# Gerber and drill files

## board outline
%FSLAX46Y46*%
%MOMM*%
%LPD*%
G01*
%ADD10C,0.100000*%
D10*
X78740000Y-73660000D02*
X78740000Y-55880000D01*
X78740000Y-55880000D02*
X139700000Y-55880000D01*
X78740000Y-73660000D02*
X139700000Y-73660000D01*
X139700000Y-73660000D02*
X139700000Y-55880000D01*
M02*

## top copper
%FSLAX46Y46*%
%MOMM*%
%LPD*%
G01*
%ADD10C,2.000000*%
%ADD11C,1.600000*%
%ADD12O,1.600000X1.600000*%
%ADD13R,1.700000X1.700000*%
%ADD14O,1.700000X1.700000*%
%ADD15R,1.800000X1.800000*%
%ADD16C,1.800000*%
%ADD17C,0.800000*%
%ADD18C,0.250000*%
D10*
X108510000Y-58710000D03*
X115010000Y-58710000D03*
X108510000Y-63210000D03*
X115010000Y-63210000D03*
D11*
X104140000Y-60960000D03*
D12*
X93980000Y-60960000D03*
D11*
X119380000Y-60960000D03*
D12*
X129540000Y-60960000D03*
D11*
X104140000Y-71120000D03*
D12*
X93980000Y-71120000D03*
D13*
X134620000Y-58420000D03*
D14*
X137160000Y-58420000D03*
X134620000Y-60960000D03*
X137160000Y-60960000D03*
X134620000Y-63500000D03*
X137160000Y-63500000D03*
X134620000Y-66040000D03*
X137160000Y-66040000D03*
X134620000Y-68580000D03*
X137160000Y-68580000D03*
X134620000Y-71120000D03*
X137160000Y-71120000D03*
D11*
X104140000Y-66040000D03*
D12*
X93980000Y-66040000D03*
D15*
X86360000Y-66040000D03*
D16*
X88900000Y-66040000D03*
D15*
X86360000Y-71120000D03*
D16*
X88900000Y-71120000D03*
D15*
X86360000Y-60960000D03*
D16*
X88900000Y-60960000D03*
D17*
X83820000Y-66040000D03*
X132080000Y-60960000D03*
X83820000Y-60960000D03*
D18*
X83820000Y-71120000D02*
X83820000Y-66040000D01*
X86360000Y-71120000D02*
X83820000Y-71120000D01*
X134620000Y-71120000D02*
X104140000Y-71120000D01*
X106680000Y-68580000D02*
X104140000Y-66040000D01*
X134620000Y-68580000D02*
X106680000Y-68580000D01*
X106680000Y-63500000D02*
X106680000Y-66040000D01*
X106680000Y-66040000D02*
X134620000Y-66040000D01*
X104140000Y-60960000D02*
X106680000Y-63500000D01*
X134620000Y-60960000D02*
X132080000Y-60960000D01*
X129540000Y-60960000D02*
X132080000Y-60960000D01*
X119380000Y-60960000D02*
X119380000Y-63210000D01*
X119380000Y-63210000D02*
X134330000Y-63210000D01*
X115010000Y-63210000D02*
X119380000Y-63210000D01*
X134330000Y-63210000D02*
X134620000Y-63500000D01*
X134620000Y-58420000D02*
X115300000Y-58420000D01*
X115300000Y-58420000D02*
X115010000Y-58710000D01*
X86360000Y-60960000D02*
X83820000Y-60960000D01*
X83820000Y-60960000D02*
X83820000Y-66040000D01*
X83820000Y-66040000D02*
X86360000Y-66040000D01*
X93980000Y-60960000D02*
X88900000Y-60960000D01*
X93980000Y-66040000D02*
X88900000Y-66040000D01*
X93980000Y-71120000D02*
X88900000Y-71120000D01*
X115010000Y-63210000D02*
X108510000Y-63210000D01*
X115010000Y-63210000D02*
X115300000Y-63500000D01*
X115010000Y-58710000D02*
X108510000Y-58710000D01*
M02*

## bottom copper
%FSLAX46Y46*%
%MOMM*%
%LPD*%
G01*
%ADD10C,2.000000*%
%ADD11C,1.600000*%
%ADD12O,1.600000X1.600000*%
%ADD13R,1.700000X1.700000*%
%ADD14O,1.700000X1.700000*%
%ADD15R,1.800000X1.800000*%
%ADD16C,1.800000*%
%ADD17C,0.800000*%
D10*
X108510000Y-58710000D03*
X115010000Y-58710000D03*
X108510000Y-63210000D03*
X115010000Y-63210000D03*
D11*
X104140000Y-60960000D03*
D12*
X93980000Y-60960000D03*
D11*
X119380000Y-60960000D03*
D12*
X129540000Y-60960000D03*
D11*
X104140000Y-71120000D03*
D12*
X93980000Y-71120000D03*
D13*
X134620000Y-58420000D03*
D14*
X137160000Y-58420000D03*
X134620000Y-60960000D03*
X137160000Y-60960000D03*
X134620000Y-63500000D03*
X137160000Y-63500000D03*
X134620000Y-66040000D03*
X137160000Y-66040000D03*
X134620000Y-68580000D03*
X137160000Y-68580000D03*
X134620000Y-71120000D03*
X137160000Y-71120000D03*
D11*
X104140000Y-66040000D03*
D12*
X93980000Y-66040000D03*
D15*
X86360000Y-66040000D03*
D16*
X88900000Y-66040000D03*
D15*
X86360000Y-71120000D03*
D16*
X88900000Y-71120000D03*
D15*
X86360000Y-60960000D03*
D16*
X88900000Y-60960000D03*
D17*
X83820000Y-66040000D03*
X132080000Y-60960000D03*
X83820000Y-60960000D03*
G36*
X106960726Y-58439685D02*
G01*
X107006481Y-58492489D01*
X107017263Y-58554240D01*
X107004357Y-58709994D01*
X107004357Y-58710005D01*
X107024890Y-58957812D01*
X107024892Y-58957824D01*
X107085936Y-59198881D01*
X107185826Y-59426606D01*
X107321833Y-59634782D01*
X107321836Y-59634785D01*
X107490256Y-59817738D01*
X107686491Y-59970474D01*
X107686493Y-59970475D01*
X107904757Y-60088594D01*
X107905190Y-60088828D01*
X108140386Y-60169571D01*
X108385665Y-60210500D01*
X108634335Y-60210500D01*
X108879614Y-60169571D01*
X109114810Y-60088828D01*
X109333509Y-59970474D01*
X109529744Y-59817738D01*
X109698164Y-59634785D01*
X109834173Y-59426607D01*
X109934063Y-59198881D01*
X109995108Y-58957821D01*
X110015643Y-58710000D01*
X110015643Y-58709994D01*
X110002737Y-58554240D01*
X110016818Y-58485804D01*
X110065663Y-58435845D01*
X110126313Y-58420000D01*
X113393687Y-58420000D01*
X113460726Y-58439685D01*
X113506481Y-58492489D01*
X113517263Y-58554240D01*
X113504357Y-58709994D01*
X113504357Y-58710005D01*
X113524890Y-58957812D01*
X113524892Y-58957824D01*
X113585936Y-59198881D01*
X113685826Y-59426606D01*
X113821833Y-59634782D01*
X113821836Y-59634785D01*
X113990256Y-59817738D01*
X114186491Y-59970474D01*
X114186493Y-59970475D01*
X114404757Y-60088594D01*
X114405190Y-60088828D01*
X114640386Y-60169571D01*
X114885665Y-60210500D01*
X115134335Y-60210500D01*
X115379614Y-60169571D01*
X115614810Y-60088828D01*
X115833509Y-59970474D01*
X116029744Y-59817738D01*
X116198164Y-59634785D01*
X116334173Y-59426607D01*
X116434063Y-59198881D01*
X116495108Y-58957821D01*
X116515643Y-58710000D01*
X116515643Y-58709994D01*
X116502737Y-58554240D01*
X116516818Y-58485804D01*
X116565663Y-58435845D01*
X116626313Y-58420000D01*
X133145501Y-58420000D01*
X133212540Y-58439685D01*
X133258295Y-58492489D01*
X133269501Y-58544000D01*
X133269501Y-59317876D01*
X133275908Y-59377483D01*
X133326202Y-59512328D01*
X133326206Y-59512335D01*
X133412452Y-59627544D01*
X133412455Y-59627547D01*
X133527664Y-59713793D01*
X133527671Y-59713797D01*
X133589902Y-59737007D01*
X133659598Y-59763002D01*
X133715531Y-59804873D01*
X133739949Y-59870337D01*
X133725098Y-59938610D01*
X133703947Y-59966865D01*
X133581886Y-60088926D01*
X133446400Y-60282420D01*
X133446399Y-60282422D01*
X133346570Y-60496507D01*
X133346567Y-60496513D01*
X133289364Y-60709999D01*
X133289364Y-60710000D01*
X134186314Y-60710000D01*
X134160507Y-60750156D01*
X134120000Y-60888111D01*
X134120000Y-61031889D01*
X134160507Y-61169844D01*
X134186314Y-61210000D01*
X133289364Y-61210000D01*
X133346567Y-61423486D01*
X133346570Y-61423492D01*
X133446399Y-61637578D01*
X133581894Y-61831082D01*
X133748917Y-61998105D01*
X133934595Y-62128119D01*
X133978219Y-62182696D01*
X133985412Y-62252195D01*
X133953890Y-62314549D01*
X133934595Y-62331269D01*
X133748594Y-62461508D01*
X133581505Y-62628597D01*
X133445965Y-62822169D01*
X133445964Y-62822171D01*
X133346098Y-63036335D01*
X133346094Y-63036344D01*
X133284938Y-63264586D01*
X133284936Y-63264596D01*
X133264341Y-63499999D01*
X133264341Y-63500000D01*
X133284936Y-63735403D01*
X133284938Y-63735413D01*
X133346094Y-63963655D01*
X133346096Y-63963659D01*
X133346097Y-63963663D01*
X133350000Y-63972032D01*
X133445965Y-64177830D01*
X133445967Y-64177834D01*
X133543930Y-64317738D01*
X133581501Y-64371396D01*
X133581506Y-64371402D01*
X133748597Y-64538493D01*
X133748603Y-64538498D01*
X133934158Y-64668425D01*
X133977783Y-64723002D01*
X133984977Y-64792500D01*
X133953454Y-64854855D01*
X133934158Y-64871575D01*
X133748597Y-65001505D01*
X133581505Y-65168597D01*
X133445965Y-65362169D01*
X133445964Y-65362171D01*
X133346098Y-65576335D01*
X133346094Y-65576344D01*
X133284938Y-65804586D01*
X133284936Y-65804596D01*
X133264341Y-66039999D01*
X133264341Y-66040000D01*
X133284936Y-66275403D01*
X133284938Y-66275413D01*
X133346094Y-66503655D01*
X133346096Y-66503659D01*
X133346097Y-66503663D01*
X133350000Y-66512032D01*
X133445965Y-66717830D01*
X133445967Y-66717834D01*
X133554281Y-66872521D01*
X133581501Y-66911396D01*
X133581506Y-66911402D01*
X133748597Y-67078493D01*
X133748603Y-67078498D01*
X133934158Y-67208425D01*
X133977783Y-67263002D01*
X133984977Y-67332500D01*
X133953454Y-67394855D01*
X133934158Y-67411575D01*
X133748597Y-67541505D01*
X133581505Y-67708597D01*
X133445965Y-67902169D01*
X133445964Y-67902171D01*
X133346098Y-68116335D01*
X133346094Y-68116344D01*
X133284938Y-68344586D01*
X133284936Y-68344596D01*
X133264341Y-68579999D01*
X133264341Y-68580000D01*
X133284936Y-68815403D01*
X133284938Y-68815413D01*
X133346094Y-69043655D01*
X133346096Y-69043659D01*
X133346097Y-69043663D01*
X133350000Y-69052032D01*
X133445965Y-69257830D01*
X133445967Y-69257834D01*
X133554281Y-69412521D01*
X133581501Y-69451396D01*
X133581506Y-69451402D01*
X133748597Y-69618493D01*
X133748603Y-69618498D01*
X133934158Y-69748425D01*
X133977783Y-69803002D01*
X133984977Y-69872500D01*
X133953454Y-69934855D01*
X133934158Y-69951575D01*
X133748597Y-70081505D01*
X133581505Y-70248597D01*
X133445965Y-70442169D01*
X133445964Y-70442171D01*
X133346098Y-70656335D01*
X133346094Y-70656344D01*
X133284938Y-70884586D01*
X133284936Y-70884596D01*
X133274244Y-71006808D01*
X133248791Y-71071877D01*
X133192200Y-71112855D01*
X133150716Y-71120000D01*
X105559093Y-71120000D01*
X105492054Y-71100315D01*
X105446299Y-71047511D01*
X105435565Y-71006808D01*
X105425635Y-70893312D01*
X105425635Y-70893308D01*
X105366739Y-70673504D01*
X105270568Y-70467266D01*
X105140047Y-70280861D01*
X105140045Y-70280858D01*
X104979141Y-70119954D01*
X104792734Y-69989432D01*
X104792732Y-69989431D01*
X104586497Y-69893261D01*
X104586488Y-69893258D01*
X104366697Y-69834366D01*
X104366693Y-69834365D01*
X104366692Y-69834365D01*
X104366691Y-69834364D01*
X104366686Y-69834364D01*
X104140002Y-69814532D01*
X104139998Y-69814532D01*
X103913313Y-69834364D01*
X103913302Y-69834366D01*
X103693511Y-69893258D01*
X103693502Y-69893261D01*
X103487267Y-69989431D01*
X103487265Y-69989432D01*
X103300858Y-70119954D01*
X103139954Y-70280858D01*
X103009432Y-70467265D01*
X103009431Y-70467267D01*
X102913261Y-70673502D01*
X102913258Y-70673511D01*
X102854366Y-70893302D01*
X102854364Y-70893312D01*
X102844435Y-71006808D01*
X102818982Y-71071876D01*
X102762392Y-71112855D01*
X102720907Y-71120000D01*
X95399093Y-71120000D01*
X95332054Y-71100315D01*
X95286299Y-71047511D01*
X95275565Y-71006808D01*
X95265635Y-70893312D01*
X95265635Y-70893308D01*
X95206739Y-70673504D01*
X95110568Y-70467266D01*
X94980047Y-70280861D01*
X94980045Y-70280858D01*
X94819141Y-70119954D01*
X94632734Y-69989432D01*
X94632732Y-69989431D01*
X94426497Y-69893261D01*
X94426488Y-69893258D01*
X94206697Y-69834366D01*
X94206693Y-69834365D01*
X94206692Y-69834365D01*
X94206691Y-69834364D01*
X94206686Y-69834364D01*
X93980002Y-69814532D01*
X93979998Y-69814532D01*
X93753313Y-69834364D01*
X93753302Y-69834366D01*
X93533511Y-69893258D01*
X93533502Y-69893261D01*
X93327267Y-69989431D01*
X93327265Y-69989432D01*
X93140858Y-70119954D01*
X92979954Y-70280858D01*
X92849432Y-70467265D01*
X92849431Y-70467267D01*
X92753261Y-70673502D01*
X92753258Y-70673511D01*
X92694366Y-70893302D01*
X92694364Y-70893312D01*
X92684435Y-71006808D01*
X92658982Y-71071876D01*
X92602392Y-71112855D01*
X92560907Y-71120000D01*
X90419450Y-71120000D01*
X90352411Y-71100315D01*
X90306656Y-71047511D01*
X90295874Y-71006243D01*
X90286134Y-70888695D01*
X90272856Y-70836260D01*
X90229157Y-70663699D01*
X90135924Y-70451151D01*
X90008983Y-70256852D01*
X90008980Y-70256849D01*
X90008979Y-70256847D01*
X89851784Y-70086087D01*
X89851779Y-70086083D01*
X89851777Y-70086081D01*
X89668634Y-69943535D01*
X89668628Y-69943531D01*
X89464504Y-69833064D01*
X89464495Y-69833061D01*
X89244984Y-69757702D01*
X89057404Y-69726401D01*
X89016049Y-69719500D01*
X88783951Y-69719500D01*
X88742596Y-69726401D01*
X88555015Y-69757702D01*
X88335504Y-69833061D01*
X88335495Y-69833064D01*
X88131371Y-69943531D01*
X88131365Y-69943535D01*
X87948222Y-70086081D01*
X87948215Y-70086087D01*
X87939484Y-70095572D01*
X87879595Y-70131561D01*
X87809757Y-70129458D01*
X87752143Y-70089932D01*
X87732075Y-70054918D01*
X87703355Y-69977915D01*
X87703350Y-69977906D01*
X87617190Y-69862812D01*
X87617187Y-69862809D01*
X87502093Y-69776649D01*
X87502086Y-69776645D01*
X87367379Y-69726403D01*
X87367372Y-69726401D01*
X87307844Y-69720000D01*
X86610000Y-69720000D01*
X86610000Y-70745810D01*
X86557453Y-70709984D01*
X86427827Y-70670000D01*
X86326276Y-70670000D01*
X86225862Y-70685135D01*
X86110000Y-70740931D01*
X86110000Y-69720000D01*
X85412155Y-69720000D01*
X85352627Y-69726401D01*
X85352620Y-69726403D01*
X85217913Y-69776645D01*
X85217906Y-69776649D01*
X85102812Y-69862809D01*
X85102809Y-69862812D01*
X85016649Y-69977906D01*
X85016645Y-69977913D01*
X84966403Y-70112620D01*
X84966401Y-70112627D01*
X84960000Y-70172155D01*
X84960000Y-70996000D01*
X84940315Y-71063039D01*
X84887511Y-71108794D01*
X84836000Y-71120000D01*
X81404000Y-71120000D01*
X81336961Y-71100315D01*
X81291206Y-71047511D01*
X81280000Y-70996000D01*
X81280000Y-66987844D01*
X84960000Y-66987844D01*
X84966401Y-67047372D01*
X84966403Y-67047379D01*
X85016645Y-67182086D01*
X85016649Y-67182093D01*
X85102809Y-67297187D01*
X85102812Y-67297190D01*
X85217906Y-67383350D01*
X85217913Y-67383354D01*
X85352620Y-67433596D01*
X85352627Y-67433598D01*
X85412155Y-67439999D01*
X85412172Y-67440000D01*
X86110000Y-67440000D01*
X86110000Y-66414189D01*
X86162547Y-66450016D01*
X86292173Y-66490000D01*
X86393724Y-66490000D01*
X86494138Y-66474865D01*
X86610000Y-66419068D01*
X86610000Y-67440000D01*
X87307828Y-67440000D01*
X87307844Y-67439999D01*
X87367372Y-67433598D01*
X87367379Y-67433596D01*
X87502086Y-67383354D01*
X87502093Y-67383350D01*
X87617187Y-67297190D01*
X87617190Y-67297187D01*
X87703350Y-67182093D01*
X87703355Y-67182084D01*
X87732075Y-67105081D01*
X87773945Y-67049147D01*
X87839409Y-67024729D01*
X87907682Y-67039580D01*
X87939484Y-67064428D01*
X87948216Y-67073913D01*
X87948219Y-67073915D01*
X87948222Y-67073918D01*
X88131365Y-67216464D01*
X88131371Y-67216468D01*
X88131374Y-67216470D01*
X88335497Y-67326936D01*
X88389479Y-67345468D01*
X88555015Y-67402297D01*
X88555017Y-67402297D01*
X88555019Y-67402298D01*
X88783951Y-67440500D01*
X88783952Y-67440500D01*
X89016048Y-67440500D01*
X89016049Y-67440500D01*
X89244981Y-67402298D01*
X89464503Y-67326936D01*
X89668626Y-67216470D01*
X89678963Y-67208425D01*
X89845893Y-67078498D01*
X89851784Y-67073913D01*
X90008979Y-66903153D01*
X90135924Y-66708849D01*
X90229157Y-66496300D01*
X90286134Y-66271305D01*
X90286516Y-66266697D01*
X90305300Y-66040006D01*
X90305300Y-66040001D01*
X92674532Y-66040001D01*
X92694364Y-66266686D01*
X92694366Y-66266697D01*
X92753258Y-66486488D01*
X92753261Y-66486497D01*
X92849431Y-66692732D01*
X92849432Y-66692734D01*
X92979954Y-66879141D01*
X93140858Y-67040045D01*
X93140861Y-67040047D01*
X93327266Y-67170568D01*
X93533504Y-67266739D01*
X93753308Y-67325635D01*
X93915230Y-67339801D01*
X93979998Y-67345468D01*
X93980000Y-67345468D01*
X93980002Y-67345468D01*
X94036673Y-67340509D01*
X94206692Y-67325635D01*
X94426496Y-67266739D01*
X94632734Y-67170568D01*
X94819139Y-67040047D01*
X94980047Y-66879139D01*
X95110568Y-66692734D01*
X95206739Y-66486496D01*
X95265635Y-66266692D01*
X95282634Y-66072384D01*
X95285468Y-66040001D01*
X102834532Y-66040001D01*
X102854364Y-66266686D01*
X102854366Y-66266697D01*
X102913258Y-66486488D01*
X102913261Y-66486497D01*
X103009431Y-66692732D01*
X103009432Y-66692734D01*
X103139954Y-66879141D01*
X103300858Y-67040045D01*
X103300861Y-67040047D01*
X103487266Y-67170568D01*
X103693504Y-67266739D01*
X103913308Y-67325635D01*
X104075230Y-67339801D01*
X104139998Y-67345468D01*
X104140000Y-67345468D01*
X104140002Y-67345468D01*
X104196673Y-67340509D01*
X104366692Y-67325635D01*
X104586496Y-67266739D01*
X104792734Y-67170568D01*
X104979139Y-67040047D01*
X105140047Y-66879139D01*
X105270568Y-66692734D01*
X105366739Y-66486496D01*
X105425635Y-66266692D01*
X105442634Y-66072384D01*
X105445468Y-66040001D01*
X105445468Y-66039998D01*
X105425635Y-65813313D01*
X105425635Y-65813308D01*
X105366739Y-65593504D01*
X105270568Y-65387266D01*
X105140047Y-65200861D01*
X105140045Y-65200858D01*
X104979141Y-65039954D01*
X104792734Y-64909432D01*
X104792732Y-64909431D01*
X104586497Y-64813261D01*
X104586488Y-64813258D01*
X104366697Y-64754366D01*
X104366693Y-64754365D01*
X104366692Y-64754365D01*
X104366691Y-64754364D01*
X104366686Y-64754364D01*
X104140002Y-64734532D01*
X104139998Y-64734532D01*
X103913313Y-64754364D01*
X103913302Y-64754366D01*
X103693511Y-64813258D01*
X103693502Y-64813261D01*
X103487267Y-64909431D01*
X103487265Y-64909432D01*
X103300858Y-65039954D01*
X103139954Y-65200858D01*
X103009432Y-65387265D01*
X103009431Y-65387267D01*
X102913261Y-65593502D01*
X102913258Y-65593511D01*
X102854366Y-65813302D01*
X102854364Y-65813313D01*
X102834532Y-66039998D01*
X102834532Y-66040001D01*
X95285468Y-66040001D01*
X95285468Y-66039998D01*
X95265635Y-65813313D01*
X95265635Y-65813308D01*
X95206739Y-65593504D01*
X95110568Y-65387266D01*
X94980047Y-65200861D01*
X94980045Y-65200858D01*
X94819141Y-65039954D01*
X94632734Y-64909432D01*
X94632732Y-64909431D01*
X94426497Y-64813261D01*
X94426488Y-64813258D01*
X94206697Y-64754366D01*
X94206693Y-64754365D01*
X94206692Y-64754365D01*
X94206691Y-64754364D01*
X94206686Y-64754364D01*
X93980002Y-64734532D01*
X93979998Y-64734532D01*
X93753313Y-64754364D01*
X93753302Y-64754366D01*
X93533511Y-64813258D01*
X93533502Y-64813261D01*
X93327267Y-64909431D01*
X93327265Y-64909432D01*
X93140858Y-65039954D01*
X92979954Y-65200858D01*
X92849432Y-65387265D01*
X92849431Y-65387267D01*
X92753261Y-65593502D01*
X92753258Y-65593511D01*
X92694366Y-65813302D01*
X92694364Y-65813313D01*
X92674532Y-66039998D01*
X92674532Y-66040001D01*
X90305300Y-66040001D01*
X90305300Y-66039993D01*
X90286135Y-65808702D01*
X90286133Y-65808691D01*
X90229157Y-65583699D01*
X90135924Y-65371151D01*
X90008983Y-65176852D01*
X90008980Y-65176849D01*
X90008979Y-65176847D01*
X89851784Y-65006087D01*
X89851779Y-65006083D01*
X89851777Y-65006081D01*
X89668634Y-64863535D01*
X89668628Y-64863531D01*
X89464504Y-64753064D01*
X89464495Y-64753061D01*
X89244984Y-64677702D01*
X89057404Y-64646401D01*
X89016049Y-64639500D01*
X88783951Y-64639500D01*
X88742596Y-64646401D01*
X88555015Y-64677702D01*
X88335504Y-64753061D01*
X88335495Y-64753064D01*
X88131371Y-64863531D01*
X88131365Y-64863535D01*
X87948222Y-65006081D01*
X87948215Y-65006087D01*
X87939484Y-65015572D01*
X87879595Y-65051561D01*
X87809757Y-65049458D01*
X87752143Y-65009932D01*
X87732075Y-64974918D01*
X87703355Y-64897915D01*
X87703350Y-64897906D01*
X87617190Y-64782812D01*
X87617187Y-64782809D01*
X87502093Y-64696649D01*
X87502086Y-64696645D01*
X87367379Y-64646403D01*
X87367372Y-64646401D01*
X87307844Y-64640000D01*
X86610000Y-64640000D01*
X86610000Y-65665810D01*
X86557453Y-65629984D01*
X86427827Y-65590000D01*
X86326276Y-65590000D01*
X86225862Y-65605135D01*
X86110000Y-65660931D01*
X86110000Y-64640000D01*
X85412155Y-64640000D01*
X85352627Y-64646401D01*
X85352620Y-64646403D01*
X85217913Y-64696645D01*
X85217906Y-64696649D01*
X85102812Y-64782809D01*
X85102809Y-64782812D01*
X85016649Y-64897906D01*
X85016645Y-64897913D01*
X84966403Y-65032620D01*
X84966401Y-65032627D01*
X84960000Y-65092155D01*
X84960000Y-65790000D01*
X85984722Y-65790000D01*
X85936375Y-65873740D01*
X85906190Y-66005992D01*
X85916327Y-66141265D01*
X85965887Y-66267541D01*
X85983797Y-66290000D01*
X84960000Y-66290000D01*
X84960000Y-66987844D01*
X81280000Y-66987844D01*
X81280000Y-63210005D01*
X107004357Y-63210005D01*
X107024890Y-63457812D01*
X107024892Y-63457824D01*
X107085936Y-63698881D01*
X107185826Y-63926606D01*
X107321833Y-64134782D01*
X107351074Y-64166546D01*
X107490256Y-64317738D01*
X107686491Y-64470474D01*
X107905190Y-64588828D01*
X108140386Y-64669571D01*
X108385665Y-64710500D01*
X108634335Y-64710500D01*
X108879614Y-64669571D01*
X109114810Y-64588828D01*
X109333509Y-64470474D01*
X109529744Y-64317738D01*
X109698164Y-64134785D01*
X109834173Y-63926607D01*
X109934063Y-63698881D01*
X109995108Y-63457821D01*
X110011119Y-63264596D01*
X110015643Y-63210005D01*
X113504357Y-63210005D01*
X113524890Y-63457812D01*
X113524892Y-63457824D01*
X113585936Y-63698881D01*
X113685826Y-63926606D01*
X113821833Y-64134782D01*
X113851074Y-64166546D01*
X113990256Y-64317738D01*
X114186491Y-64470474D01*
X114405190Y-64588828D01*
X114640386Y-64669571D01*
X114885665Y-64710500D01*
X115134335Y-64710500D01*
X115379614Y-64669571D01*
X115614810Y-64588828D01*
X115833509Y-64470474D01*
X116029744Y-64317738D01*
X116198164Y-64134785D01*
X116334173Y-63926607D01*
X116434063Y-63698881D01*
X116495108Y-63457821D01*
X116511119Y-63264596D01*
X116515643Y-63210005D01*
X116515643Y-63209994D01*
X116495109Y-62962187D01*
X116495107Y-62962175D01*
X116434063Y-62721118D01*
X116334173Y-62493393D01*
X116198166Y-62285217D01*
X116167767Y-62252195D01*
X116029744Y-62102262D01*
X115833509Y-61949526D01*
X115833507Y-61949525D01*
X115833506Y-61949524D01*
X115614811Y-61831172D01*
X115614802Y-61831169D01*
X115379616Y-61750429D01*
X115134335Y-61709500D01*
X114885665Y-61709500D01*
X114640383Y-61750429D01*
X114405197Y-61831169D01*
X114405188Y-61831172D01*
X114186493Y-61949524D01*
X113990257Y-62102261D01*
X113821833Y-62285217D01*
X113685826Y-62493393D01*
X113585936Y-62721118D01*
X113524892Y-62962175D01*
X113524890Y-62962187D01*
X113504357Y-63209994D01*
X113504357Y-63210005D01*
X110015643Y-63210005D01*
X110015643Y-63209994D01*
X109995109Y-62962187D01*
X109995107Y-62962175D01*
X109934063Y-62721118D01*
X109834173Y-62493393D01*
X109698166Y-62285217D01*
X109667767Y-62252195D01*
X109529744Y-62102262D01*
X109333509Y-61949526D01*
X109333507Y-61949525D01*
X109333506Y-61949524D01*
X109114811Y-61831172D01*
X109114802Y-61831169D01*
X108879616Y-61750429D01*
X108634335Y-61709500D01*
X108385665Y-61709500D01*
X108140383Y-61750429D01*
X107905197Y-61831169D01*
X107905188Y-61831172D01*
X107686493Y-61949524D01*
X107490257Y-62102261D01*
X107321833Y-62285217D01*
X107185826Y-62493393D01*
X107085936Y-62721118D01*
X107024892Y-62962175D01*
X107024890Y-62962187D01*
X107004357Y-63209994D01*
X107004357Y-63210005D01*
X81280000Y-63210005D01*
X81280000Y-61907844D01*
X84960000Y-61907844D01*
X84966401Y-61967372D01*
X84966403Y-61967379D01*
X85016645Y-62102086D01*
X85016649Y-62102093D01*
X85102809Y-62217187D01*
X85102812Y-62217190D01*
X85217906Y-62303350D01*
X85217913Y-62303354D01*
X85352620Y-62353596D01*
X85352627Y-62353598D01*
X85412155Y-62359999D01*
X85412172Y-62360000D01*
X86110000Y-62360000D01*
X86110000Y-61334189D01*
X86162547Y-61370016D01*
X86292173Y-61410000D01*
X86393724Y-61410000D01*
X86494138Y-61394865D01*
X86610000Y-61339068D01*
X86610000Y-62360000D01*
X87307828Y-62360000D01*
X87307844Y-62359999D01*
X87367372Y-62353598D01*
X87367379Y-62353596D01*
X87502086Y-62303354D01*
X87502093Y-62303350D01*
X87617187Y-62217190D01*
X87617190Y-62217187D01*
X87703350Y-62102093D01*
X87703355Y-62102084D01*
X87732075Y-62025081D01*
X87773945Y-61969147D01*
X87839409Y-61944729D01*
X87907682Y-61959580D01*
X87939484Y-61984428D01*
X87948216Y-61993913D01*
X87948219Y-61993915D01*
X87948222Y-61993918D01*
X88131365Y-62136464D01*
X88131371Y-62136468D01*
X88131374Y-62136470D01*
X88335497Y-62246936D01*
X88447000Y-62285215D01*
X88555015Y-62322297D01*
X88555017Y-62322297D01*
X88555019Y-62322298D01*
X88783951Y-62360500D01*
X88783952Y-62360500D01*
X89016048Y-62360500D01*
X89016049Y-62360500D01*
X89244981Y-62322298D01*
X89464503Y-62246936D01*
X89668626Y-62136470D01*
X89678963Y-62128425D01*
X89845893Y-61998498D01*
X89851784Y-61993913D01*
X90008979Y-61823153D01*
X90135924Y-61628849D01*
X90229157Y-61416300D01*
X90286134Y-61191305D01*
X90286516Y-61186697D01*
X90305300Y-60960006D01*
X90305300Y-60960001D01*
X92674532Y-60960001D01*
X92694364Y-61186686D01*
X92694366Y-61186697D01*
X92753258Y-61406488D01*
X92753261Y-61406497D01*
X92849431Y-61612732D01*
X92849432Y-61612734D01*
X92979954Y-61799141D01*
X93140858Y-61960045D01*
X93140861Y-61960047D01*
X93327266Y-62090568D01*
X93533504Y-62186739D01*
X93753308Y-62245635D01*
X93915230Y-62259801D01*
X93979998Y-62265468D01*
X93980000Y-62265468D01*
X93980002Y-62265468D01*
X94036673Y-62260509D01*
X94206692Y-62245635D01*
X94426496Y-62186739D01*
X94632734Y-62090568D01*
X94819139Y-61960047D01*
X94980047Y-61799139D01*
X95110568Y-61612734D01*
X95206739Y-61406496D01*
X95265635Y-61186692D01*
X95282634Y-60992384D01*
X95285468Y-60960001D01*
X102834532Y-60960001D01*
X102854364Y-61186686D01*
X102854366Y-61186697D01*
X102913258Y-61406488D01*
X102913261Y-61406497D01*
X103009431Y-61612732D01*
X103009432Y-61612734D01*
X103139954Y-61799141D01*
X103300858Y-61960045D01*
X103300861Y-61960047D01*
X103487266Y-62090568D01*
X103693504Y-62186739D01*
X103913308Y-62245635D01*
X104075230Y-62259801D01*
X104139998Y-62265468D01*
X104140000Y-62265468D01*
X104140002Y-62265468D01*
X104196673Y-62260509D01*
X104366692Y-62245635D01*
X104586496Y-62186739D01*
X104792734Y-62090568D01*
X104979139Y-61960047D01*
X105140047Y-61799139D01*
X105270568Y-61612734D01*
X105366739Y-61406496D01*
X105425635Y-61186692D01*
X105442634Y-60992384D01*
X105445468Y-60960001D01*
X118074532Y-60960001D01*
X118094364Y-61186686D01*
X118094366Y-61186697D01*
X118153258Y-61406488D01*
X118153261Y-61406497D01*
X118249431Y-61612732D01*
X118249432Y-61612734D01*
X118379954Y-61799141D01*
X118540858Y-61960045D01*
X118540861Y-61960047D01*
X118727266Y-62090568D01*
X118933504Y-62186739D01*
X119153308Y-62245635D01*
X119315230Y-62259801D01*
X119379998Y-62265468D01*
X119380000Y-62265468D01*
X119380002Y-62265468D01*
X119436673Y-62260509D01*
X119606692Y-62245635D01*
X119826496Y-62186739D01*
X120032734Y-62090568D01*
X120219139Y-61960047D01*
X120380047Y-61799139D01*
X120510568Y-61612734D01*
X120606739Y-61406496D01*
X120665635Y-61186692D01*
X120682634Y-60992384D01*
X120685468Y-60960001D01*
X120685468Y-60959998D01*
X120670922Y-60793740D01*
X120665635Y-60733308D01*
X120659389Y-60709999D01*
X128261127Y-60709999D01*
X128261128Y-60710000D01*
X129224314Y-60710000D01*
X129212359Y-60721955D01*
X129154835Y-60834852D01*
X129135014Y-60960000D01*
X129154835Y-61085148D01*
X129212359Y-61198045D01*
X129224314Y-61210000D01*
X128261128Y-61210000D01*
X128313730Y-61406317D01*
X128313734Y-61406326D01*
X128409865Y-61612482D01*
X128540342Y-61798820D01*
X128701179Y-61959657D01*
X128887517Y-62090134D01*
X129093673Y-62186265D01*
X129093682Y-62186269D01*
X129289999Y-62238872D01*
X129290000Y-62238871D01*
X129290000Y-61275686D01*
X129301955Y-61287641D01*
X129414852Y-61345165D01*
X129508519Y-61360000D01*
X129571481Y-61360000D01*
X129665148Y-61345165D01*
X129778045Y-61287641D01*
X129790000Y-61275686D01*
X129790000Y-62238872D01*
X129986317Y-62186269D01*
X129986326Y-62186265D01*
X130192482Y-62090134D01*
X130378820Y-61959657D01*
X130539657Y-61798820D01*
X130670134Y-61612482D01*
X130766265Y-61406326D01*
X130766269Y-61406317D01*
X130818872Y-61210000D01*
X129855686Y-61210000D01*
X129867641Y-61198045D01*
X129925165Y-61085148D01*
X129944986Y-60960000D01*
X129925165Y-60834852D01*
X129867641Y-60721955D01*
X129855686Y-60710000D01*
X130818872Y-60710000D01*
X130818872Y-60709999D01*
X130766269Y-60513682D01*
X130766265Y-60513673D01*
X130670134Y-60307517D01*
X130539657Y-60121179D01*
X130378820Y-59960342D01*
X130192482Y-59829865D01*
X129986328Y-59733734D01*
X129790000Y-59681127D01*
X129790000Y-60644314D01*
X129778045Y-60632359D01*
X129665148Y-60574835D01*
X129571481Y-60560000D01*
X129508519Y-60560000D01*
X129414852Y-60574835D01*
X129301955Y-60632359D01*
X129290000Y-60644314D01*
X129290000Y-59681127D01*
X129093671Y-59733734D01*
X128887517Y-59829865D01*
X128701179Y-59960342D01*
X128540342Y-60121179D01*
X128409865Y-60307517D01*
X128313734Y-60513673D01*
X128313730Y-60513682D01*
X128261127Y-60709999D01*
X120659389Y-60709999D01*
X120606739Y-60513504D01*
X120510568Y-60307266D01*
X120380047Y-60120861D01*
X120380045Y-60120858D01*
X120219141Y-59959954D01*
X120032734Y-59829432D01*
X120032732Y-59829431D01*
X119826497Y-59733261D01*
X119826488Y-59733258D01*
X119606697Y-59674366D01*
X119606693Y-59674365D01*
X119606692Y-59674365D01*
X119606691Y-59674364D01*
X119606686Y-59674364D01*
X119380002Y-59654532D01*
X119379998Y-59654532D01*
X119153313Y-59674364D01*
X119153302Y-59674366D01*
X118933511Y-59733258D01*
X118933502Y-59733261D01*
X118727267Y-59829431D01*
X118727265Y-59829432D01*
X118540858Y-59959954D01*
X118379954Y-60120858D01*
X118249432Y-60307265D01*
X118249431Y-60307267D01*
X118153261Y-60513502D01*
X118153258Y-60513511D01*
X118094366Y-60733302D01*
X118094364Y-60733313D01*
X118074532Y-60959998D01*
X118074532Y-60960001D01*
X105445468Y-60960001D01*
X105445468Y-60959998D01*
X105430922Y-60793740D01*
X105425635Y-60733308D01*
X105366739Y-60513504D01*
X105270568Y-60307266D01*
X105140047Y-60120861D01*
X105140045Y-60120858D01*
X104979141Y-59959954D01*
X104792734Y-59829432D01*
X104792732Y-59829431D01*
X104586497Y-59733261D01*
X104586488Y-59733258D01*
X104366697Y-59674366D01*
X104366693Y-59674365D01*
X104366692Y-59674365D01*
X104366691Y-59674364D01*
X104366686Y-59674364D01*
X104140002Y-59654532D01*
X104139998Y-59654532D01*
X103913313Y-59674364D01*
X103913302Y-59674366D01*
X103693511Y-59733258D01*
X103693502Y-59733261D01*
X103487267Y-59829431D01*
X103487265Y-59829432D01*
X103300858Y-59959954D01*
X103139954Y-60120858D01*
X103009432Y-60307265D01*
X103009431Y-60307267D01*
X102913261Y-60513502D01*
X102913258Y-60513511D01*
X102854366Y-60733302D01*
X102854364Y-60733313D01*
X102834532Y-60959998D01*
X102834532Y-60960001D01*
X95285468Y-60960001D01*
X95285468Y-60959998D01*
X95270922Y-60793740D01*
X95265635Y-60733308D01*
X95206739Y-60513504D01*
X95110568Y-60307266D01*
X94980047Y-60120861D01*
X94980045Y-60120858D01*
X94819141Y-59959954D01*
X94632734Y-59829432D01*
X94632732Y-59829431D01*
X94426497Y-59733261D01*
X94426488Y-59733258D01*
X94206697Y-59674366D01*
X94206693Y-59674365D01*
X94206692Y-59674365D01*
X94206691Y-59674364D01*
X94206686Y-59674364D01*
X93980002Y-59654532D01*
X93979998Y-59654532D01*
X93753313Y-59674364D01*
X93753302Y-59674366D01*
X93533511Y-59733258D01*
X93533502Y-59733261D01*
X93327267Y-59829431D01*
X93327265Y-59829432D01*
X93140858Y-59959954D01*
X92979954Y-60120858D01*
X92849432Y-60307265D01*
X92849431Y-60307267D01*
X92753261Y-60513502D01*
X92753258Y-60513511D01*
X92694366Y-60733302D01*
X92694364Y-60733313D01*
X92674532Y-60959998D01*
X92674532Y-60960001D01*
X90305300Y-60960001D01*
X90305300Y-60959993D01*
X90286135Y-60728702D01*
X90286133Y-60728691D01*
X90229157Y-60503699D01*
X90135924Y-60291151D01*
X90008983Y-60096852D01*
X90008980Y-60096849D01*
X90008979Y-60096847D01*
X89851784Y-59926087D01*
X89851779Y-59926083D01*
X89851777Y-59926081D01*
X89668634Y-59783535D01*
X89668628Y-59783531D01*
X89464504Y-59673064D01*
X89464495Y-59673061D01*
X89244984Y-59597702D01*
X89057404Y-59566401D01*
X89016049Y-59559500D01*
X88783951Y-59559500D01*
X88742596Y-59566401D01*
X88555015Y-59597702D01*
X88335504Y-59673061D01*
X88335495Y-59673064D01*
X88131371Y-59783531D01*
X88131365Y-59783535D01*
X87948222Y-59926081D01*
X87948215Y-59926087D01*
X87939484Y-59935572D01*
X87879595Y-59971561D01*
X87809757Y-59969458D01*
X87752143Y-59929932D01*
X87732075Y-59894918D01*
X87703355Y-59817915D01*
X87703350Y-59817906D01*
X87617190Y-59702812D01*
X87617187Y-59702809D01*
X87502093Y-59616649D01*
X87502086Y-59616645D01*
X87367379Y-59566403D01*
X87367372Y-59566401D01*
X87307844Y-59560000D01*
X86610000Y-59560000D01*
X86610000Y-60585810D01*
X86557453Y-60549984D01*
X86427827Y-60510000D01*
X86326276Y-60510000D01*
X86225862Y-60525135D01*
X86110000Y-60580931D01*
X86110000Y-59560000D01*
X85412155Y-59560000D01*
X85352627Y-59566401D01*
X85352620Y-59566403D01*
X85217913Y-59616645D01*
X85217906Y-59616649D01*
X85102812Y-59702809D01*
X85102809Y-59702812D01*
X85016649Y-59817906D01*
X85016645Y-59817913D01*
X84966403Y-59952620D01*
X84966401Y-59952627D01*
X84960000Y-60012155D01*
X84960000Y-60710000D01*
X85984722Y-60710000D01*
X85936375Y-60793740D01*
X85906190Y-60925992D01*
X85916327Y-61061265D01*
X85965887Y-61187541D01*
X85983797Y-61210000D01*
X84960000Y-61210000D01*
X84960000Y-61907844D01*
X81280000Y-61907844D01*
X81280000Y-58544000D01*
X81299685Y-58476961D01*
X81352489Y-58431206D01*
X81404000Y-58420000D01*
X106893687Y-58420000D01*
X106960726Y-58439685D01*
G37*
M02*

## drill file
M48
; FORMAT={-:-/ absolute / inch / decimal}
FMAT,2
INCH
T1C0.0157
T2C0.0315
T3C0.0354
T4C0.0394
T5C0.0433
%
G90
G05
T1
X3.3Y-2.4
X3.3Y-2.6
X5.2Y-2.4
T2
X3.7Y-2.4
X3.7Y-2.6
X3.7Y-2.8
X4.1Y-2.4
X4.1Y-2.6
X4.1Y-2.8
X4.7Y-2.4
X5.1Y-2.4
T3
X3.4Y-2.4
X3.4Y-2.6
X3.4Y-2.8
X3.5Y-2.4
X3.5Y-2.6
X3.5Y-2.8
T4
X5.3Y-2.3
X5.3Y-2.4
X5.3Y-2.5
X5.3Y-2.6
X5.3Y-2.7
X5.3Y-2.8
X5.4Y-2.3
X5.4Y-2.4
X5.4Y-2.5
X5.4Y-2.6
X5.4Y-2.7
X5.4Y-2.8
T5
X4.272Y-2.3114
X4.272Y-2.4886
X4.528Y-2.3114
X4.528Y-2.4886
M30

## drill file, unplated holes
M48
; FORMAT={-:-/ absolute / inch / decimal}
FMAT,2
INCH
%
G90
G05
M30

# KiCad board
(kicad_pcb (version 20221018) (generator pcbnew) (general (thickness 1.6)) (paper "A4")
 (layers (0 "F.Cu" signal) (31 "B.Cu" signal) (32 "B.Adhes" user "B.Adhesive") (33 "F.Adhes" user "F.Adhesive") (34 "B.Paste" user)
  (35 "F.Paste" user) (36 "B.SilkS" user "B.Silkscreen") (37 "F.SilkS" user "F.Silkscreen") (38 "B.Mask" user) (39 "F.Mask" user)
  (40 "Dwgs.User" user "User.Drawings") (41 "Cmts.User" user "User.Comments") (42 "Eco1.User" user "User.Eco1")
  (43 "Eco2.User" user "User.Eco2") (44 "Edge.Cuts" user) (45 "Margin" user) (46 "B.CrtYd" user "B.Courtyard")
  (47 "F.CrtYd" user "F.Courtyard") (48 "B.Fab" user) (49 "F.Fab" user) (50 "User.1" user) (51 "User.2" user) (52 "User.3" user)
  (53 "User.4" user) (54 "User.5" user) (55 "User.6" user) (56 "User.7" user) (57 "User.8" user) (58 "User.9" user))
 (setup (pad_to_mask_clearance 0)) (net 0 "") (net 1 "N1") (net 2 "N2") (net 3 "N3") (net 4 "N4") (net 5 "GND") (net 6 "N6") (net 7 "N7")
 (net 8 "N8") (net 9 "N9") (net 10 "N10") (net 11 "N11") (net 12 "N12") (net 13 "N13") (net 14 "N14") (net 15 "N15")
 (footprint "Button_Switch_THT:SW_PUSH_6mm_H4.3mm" (layer "F.Cu") (at 108.51 58.71)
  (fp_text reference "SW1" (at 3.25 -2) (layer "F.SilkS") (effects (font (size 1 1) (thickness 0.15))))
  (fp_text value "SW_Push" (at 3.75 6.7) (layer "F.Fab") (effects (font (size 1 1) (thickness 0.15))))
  (pad "1" thru_hole circle (at 0 0 90) (size 2 2) (drill 1.1) (layers "*.Cu" "*.Mask") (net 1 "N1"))
  (pad "1" thru_hole circle (at 6.5 0 90) (size 2 2) (drill 1.1) (layers "*.Cu" "*.Mask") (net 1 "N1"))
  (pad "2" thru_hole circle (at 0 4.5 90) (size 2 2) (drill 1.1) (layers "*.Cu" "*.Mask") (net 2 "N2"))
  (pad "2" thru_hole circle (at 6.5 4.5 90) (size 2 2) (drill 1.1) (layers "*.Cu" "*.Mask") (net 2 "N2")))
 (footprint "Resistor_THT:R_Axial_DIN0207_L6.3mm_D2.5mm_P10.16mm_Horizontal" (layer "F.Cu") (at 104.14 60.96 180)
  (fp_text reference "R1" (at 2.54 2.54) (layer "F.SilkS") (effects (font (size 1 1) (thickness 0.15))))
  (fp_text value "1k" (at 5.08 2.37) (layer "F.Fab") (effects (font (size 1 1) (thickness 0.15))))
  (pad "1" thru_hole circle (at 0 0 180) (size 1.6 1.6) (drill 0.8) (layers "*.Cu" "*.Mask") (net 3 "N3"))
  (pad "2" thru_hole oval (at 10.16 0 180) (size 1.6 1.6) (drill 0.8) (layers "*.Cu" "*.Mask") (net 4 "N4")))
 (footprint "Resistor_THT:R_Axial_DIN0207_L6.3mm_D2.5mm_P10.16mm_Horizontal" (layer "F.Cu") (at 119.38 60.96)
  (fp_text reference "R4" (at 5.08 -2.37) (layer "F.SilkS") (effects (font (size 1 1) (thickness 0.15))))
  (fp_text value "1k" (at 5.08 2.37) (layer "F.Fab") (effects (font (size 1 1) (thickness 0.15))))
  (pad "1" thru_hole circle (at 0 0) (size 1.6 1.6) (drill 0.8) (layers "*.Cu" "*.Mask") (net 2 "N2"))
  (pad "2" thru_hole oval (at 10.16 0) (size 1.6 1.6) (drill 0.8) (layers "*.Cu" "*.Mask") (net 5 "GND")))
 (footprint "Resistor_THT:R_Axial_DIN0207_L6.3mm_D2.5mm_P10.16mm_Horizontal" (layer "F.Cu") (at 104.14 71.12 180)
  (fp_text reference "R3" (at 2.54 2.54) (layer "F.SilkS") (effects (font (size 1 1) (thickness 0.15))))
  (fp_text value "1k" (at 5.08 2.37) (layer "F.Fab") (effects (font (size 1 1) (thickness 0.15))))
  (pad "1" thru_hole circle (at 0 0 180) (size 1.6 1.6) (drill 0.8) (layers "*.Cu" "*.Mask") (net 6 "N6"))
  (pad "2" thru_hole oval (at 10.16 0 180) (size 1.6 1.6) (drill 0.8) (layers "*.Cu" "*.Mask") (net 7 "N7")))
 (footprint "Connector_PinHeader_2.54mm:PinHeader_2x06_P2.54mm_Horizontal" (layer "F.Cu") (at 134.62 58.42)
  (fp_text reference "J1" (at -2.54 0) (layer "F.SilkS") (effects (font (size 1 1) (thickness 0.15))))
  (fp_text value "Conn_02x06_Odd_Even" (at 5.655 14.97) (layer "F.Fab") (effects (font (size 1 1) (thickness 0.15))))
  (pad "1" thru_hole rect (at 0 0) (size 1.7 1.7) (drill 1) (layers "*.Cu" "*.Mask") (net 1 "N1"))
  (pad "2" thru_hole oval (at 2.54 0) (size 1.7 1.7) (drill 1) (layers "*.Cu" "*.Mask") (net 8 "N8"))
  (pad "3" thru_hole oval (at 0 2.54) (size 1.7 1.7) (drill 1) (layers "*.Cu" "*.Mask") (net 5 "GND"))
  (pad "4" thru_hole oval (at 2.54 2.54) (size 1.7 1.7) (drill 1) (layers "*.Cu" "*.Mask") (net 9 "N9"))
  (pad "5" thru_hole oval (at 0 5.08) (size 1.7 1.7) (drill 1) (layers "*.Cu" "*.Mask") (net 2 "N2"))
  (pad "6" thru_hole oval (at 2.54 5.08) (size 1.7 1.7) (drill 1) (layers "*.Cu" "*.Mask") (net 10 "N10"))
  (pad "7" thru_hole oval (at 0 7.62) (size 1.7 1.7) (drill 1) (layers "*.Cu" "*.Mask") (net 3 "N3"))
  (pad "8" thru_hole oval (at 2.54 7.62) (size 1.7 1.7) (drill 1) (layers "*.Cu" "*.Mask") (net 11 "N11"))
  (pad "9" thru_hole oval (at 0 10.16) (size 1.7 1.7) (drill 1) (layers "*.Cu" "*.Mask") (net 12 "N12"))
  (pad "10" thru_hole oval (at 2.54 10.16) (size 1.7 1.7) (drill 1) (layers "*.Cu" "*.Mask") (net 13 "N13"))
  (pad "11" thru_hole oval (at 0 12.7) (size 1.7 1.7) (drill 1) (layers "*.Cu" "*.Mask") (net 6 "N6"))
  (pad "12" thru_hole oval (at 2.54 12.7) (size 1.7 1.7) (drill 1) (layers "*.Cu" "*.Mask") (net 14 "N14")))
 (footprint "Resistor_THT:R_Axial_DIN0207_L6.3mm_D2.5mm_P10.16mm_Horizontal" (layer "F.Cu") (at 104.14 66.04 180)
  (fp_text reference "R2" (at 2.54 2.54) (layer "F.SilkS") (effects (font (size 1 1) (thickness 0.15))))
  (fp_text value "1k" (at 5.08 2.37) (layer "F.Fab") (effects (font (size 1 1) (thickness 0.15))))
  (pad "1" thru_hole circle (at 0 0 180) (size 1.6 1.6) (drill 0.8) (layers "*.Cu" "*.Mask") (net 12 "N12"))
  (pad "2" thru_hole oval (at 10.16 0 180) (size 1.6 1.6) (drill 0.8) (layers "*.Cu" "*.Mask") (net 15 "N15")))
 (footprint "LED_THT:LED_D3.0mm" (layer "F.Cu") (at 86.36 66.04)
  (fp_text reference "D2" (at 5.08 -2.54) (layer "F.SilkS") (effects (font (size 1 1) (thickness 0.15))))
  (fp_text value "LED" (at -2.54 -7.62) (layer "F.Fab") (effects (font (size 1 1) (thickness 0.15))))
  (pad "1" thru_hole rect (at 0 0) (size 1.8 1.8) (drill 0.9) (layers "*.Cu" "*.Mask") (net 5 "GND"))
  (pad "2" thru_hole circle (at 2.54 0) (size 1.8 1.8) (drill 0.9) (layers "*.Cu" "*.Mask") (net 15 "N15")))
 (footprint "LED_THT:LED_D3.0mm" (layer "F.Cu") (at 86.36 71.12)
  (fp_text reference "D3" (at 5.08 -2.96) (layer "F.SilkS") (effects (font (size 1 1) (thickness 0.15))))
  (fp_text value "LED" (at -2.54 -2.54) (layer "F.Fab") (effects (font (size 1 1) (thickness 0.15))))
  (pad "1" thru_hole rect (at 0 0) (size 1.8 1.8) (drill 0.9) (layers "*.Cu" "*.Mask") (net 5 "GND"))
  (pad "2" thru_hole circle (at 2.54 0) (size 1.8 1.8) (drill 0.9) (layers "*.Cu" "*.Mask") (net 7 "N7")))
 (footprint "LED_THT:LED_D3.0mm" (layer "F.Cu") (at 86.36 60.96)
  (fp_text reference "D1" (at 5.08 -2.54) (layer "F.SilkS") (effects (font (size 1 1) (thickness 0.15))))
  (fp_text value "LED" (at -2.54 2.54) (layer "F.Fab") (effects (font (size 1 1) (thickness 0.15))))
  (pad "1" thru_hole rect (at 0 0) (size 1.8 1.8) (drill 0.9) (layers "*.Cu" "*.Mask") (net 5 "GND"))
  (pad "2" thru_hole circle (at 2.54 0) (size 1.8 1.8) (drill 0.9) (layers "*.Cu" "*.Mask") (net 4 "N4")))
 (gr_line (start 78.74 55.88) (end 139.7 55.88) (stroke (width 0.1) (type default)) (layer "Edge.Cuts"))
 (gr_line (start 78.74 73.66) (end 78.74 55.88) (stroke (width 0.1) (type default)) (layer "Edge.Cuts"))
 (gr_line (start 78.74 73.66) (end 139.7 73.66) (stroke (width 0.1) (type default)) (layer "Edge.Cuts"))
 (gr_line (start 139.7 73.66) (end 139.7 55.88) (stroke (width 0.1) (type default)) (layer "Edge.Cuts"))
 (segment (start 86.36 71.12) (end 83.82 71.12) (width 0.25) (layer "F.Cu") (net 5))
 (segment (start 134.62 60.96) (end 132.08 60.96) (width 0.25) (layer "F.Cu") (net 5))
 (segment (start 86.36 60.96) (end 83.82 60.96) (width 0.25) (layer "F.Cu") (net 5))
 (segment (start 83.82 71.12) (end 83.82 66.04) (width 0.25) (layer "F.Cu") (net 5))
 (segment (start 129.54 60.96) (end 132.08 60.96) (width 0.25) (layer "F.Cu") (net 5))
 (segment (start 83.82 60.96) (end 83.82 66.04) (width 0.25) (layer "F.Cu") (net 5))
 (segment (start 83.82 66.04) (end 86.36 66.04) (width 0.25) (layer "F.Cu") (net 5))
 (via (at 132.08 60.96) (size 0.8) (drill 0.4) (layers "F.Cu" "B.Cu") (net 5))
 (via (at 83.82 66.04) (size 0.8) (drill 0.4) (layers "F.Cu" "B.Cu") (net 5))
 (via (at 83.82 60.96) (size 0.8) (drill 0.4) (layers "F.Cu" "B.Cu") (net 5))
 (segment (start 93.98 60.96) (end 88.9 60.96) (width 0.25) (layer "F.Cu") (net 4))
 (segment (start 93.98 66.04) (end 88.9 66.04) (width 0.25) (layer "F.Cu") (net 15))
 (segment (start 93.98 71.12) (end 88.9 71.12) (width 0.25) (layer "F.Cu") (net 7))
 (segment (start 115.01 58.71) (end 108.51 58.71) (width 0.25) (layer "F.Cu") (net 1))
 (segment (start 134.62 58.42) (end 115.3 58.42) (width 0.25) (layer "F.Cu") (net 1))
 (segment (start 115.3 58.42) (end 115.01 58.71) (width 0.25) (layer "F.Cu") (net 1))
 (segment (start 106.68 68.58) (end 104.14 66.04) (width 0.25) (layer "F.Cu") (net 12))
 (segment (start 134.62 68.58) (end 106.68 68.58) (width 0.25) (layer "F.Cu") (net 12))
 (segment (start 119.38 63.21) (end 134.33 63.21) (width 0.25) (layer "F.Cu") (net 2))
 (segment (start 119.38 60.96) (end 119.38 63.21) (width 0.25) (layer "F.Cu") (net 2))
 (segment (start 115.01 63.21) (end 119.38 63.21) (width 0.25) (layer "F.Cu") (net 2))
 (segment (start 115.01 63.21) (end 108.51 63.21) (width 0.25) (layer "F.Cu") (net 2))
 (segment (start 134.33 63.21) (end 134.62 63.5) (width 0.25) (layer "F.Cu") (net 2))
 (segment (start 115.01 63.21) (end 115.3 63.5) (width 0.25) (layer "F.Cu") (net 2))
 (segment (start 106.68 66.04) (end 134.62 66.04) (width 0.25) (layer "F.Cu") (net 3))
 (segment (start 104.14 60.96) (end 106.68 63.5) (width 0.25) (layer "F.Cu") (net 3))
 (segment (start 106.68 63.5) (end 106.68 66.04) (width 0.25) (layer "F.Cu") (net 3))
 (segment (start 134.62 71.12) (end 104.14 71.12) (width 0.25) (layer "F.Cu") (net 6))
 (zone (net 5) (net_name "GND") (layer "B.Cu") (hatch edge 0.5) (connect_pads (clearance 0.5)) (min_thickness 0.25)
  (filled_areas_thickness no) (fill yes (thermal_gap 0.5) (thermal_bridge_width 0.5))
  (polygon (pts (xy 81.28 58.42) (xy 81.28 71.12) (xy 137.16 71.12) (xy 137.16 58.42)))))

